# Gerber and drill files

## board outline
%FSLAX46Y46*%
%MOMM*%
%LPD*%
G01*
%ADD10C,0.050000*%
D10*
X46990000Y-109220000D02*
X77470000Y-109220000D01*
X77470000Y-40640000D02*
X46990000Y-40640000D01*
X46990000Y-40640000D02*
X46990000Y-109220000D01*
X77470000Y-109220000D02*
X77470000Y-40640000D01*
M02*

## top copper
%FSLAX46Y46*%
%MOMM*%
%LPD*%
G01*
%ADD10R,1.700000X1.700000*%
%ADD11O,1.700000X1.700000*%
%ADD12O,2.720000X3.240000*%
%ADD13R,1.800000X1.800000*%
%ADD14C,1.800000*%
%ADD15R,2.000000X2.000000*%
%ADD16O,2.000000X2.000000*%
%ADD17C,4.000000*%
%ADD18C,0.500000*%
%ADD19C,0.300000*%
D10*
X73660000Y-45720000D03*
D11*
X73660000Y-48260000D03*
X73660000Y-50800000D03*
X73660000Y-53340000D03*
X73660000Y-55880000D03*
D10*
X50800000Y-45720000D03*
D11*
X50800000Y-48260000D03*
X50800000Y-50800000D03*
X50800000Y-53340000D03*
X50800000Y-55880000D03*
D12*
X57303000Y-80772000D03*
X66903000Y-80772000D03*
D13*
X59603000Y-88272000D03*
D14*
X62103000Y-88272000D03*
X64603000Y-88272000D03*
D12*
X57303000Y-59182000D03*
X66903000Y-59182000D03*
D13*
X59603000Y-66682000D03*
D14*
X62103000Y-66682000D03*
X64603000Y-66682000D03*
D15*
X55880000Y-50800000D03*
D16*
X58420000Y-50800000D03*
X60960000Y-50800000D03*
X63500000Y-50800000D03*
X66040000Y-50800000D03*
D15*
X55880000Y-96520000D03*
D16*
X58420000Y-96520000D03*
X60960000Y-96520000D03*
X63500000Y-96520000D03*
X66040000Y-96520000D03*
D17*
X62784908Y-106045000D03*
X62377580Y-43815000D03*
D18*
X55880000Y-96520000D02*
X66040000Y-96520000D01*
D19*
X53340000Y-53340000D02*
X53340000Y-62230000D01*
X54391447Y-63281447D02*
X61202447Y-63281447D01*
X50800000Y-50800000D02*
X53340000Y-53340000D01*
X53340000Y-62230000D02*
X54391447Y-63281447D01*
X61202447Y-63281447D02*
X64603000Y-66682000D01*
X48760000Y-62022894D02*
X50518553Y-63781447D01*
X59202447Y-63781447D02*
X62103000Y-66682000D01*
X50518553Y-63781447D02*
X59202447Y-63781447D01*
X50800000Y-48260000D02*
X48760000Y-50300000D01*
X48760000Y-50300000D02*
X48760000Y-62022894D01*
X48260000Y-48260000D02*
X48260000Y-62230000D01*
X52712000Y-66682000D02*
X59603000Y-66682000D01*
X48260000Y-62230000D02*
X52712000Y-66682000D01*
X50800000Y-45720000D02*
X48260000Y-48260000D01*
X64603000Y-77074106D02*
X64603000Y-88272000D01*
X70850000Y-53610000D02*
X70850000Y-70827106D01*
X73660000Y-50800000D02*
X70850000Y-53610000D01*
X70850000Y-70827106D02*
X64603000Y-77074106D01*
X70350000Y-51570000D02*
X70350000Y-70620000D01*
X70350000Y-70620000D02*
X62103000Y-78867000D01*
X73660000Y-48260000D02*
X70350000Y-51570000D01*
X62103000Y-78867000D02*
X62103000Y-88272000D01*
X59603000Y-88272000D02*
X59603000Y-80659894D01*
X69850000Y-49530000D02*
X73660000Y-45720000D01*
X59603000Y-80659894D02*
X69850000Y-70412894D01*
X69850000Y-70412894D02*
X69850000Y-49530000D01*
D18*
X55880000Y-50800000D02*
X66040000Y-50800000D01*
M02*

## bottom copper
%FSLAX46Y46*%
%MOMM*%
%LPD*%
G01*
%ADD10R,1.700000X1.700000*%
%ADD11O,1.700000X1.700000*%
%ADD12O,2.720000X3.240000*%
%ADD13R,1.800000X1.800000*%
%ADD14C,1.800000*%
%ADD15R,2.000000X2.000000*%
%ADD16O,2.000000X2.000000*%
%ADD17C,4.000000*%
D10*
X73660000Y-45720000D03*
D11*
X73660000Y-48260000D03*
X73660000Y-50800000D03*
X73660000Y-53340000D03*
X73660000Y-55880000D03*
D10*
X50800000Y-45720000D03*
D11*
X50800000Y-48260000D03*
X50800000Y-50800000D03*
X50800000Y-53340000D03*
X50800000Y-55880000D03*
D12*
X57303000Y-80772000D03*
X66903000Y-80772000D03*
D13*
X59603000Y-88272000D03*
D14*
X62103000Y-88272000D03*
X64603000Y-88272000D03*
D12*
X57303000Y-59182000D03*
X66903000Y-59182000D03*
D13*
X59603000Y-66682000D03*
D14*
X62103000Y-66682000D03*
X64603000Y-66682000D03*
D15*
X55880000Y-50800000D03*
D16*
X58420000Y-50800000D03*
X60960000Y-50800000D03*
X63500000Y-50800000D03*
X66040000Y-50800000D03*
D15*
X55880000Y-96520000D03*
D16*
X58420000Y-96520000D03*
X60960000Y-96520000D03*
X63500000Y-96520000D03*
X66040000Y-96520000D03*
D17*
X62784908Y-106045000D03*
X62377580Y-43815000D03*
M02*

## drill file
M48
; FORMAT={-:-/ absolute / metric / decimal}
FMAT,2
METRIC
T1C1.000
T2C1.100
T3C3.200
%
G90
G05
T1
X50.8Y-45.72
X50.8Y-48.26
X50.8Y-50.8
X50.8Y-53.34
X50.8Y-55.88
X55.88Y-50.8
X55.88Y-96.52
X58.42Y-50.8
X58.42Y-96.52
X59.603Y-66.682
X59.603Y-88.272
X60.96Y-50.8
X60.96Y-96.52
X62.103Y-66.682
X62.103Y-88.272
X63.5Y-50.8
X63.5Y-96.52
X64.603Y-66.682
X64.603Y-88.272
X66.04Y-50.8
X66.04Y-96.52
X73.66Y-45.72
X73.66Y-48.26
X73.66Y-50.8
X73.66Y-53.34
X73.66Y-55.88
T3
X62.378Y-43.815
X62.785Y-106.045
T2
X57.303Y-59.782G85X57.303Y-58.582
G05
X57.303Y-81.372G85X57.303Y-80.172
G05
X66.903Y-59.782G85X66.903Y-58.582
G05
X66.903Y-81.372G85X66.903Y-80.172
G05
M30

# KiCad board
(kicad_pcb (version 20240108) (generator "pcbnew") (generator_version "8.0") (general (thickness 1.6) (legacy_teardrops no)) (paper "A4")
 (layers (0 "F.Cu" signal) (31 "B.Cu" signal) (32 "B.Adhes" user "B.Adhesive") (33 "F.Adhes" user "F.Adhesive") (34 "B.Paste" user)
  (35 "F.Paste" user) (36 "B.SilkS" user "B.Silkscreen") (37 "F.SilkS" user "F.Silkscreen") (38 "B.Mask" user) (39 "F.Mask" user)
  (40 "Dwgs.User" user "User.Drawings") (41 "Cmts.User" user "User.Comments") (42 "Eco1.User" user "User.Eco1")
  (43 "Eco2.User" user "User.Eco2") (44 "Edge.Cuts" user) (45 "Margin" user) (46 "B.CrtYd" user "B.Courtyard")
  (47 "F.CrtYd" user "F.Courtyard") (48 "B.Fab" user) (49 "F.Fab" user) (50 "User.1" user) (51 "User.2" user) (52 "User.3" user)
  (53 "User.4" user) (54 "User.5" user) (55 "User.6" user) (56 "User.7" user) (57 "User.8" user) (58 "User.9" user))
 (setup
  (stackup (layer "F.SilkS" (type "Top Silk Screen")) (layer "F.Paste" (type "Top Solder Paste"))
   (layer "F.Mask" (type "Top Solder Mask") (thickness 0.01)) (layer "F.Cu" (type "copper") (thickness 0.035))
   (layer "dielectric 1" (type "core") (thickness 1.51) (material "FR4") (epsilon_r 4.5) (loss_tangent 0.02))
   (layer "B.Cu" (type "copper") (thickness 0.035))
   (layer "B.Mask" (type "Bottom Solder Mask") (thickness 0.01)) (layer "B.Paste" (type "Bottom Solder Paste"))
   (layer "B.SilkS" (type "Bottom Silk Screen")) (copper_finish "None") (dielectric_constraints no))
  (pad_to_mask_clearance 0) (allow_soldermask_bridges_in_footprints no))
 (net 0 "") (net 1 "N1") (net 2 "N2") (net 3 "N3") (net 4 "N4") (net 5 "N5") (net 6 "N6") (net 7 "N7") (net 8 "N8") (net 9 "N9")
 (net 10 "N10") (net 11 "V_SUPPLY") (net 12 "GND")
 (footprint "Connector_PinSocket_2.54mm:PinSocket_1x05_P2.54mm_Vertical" (layer "F.Cu") (at 73.66 45.72)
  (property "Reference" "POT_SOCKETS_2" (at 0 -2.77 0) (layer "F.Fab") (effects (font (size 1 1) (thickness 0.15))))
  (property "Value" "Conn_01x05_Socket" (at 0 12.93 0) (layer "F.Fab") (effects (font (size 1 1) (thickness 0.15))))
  (pad "1" thru_hole rect (at 0 0) (size 1.7 1.7) (drill 1) (layers "*.Cu" "*.Mask") (remove_unused_layers no) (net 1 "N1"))
  (pad "2" thru_hole oval (at 0 2.54) (size 1.7 1.7) (drill 1) (layers "*.Cu" "*.Mask") (remove_unused_layers no) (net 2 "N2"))
  (pad "3" thru_hole oval (at 0 5.08) (size 1.7 1.7) (drill 1) (layers "*.Cu" "*.Mask") (remove_unused_layers no) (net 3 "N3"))
  (pad "4" thru_hole oval (at 0 7.62) (size 1.7 1.7) (drill 1) (layers "*.Cu" "*.Mask") (remove_unused_layers no) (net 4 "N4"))
  (pad "5" thru_hole oval (at 0 10.16) (size 1.7 1.7) (drill 1) (layers "*.Cu" "*.Mask") (remove_unused_layers no) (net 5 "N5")))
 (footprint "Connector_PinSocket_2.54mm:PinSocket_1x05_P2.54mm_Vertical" (layer "F.Cu") (at 50.8 45.72)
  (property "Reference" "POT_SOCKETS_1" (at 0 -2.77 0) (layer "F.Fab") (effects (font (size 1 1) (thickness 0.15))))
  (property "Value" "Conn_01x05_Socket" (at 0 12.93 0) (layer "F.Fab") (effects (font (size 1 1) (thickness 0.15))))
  (pad "1" thru_hole rect (at 0 0) (size 1.7 1.7) (drill 1) (layers "*.Cu" "*.Mask") (remove_unused_layers no) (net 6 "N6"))
  (pad "2" thru_hole oval (at 0 2.54) (size 1.7 1.7) (drill 1) (layers "*.Cu" "*.Mask") (remove_unused_layers no) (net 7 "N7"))
  (pad "3" thru_hole oval (at 0 5.08) (size 1.7 1.7) (drill 1) (layers "*.Cu" "*.Mask") (remove_unused_layers no) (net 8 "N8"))
  (pad "4" thru_hole oval (at 0 7.62) (size 1.7 1.7) (drill 1) (layers "*.Cu" "*.Mask") (remove_unused_layers no) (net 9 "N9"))
  (pad "5" thru_hole oval (at 0 10.16) (size 1.7 1.7) (drill 1) (layers "*.Cu" "*.Mask") (remove_unused_layers no) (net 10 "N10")))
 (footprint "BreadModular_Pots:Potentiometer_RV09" (layer "F.Cu") (at 62.23 81.28)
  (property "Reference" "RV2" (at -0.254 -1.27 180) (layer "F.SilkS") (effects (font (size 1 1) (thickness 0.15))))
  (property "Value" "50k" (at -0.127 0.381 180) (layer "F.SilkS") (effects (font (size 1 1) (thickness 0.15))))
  (pad "" thru_hole oval (at -4.927 -0.508 180) (size 2.72 3.24) (drill oval 1.1 2.3) (layers "*.Cu" "*.Mask") (remove_unused_layers no))
  (pad "" thru_hole oval (at 4.673 -0.508 180) (size 2.72 3.24) (drill oval 1.1 2.3) (layers "*.Cu" "*.Mask") (remove_unused_layers no))
  (pad "1" thru_hole rect (at -2.627 6.992 180) (size 1.8 1.8) (drill 1) (layers "*.Cu" "*.Mask") (remove_unused_layers no) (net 1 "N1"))
  (pad "2" thru_hole circle (at -0.127 6.992 180) (size 1.8 1.8) (drill 1) (layers "*.Cu" "*.Mask") (remove_unused_layers no) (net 2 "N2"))
  (pad "3" thru_hole circle (at 2.373 6.992 180) (size 1.8 1.8) (drill 1) (layers "*.Cu" "*.Mask") (remove_unused_layers no) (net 3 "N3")))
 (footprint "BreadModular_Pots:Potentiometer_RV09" (layer "F.Cu") (at 62.23 59.69)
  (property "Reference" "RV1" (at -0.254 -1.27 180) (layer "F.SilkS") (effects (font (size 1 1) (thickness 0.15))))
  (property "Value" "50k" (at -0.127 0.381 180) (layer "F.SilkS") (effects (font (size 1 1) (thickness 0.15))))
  (pad "" thru_hole oval (at -4.927 -0.508 180) (size 2.72 3.24) (drill oval 1.1 2.3) (layers "*.Cu" "*.Mask") (remove_unused_layers no))
  (pad "" thru_hole oval (at 4.673 -0.508 180) (size 2.72 3.24) (drill oval 1.1 2.3) (layers "*.Cu" "*.Mask") (remove_unused_layers no))
  (pad "1" thru_hole rect (at -2.627 6.992 180) (size 1.8 1.8) (drill 1) (layers "*.Cu" "*.Mask") (remove_unused_layers no) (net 6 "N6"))
  (pad "2" thru_hole circle (at -0.127 6.992 180) (size 1.8 1.8) (drill 1) (layers "*.Cu" "*.Mask") (remove_unused_layers no) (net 7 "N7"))
  (pad "3" thru_hole circle (at 2.373 6.992 180) (size 1.8 1.8) (drill 1) (layers "*.Cu" "*.Mask") (remove_unused_layers no) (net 8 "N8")))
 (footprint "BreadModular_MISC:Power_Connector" (layer "B.Cu") (at 55.88 50.8 -90)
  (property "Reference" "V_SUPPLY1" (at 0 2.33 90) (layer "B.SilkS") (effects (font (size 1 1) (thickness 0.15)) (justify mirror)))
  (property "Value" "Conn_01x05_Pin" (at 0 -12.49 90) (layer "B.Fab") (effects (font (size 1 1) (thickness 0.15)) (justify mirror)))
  (pad "1" thru_hole rect (at 0 0 270) (size 2 2) (drill 1) (layers "*.Cu" "*.Mask") (remove_unused_layers no) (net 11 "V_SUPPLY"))
  (pad "2" thru_hole oval (at 0 -2.54 270) (size 2 2) (drill 1) (layers "*.Cu" "*.Mask") (remove_unused_layers no) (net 11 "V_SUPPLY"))
  (pad "3" thru_hole oval (at 0 -5.08 270) (size 2 2) (drill 1) (layers "*.Cu" "*.Mask") (remove_unused_layers no) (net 11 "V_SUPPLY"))
  (pad "4" thru_hole oval (at 0 -7.62 270) (size 2 2) (drill 1) (layers "*.Cu" "*.Mask") (remove_unused_layers no) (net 11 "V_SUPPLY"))
  (pad "5" thru_hole oval (at 0 -10.16 270) (size 2 2) (drill 1) (layers "*.Cu" "*.Mask") (remove_unused_layers no) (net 11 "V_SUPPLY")))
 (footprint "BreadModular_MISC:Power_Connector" (layer "B.Cu") (at 55.88 96.52 -90)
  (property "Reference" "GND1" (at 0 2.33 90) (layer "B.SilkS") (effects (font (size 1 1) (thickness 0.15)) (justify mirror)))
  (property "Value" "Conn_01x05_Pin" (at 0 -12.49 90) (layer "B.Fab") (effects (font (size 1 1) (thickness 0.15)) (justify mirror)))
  (pad "1" thru_hole rect (at 0 0 270) (size 2 2) (drill 1) (layers "*.Cu" "*.Mask") (remove_unused_layers no) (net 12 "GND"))
  (pad "2" thru_hole oval (at 0 -2.54 270) (size 2 2) (drill 1) (layers "*.Cu" "*.Mask") (remove_unused_layers no) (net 12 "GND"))
  (pad "3" thru_hole oval (at 0 -5.08 270) (size 2 2) (drill 1) (layers "*.Cu" "*.Mask") (remove_unused_layers no) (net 12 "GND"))
  (pad "4" thru_hole oval (at 0 -7.62 270) (size 2 2) (drill 1) (layers "*.Cu" "*.Mask") (remove_unused_layers no) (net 12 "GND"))
  (pad "5" thru_hole oval (at 0 -10.16 270) (size 2 2) (drill 1) (layers "*.Cu" "*.Mask") (remove_unused_layers no) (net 12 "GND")))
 (gr_line (start 46.99 109.22) (end 77.47 109.22) (stroke (width 0.05) (type default)) (layer "Edge.Cuts"))
 (gr_line (start 77.47 40.64) (end 46.99 40.64) (stroke (width 0.05) (type default)) (layer "Edge.Cuts"))
 (gr_line (start 46.99 40.64) (end 46.99 109.22) (stroke (width 0.05) (type default)) (layer "Edge.Cuts"))
 (gr_line (start 77.47 109.22) (end 77.47 40.64) (stroke (width 0.05) (type default)) (layer "Edge.Cuts"))
 (via (at 62.784908 106.045) (size 4) (drill 3.2) (layers "F.Cu" "B.Cu") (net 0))
 (via (at 62.37758 43.815) (size 4) (drill 3.2) (layers "F.Cu" "B.Cu") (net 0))
 (segment (start 55.88 96.52) (end 66.04 96.52) (width 0.5) (layer "F.Cu") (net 12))
 (segment (start 53.34 53.34) (end 53.34 62.23) (width 0.3) (layer "F.Cu") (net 8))
 (segment (start 54.391447 63.281447) (end 61.202447 63.281447) (width 0.3) (layer "F.Cu") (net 8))
 (segment (start 50.8 50.8) (end 53.34 53.34) (width 0.3) (layer "F.Cu") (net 8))
 (segment (start 53.34 62.23) (end 54.391447 63.281447) (width 0.3) (layer "F.Cu") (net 8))
 (segment (start 61.202447 63.281447) (end 64.603 66.682) (width 0.3) (layer "F.Cu") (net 8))
 (segment (start 48.76 62.022894) (end 50.518553 63.781447) (width 0.3) (layer "F.Cu") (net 7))
 (segment (start 59.202447 63.781447) (end 62.103 66.682) (width 0.3) (layer "F.Cu") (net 7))
 (segment (start 50.518553 63.781447) (end 59.202447 63.781447) (width 0.3) (layer "F.Cu") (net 7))
 (segment (start 50.8 48.26) (end 48.76 50.3) (width 0.3) (layer "F.Cu") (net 7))
 (segment (start 48.76 50.3) (end 48.76 62.022894) (width 0.3) (layer "F.Cu") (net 7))
 (segment (start 48.26 48.26) (end 48.26 62.23) (width 0.3) (layer "F.Cu") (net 6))
 (segment (start 52.712 66.682) (end 59.603 66.682) (width 0.3) (layer "F.Cu") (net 6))
 (segment (start 48.26 62.23) (end 52.712 66.682) (width 0.3) (layer "F.Cu") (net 6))
 (segment (start 50.8 45.72) (end 48.26 48.26) (width 0.3) (layer "F.Cu") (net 6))
 (segment (start 64.603 77.074106) (end 64.603 88.272) (width 0.3) (layer "F.Cu") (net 3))
 (segment (start 70.85 53.61) (end 70.85 70.827106) (width 0.3) (layer "F.Cu") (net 3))
 (segment (start 73.66 50.8) (end 70.85 53.61) (width 0.3) (layer "F.Cu") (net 3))
 (segment (start 70.85 70.827106) (end 64.603 77.074106) (width 0.3) (layer "F.Cu") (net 3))
 (segment (start 70.35 51.57) (end 70.35 70.62) (width 0.3) (layer "F.Cu") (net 2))
 (segment (start 70.35 70.62) (end 62.103 78.867) (width 0.3) (layer "F.Cu") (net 2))
 (segment (start 73.66 48.26) (end 70.35 51.57) (width 0.3) (layer "F.Cu") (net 2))
 (segment (start 62.103 78.867) (end 62.103 88.272) (width 0.3) (layer "F.Cu") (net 2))
 (segment (start 59.603 88.272) (end 59.603 80.659894) (width 0.3) (layer "F.Cu") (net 1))
 (segment (start 69.85 49.53) (end 73.66 45.72) (width 0.3) (layer "F.Cu") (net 1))
 (segment (start 59.603 80.659894) (end 69.85 70.412894) (width 0.3) (layer "F.Cu") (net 1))
 (segment (start 69.85 70.412894) (end 69.85 49.53) (width 0.3) (layer "F.Cu") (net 1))
 (segment (start 55.88 50.8) (end 66.04 50.8) (width 0.5) (layer "F.Cu") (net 11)))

